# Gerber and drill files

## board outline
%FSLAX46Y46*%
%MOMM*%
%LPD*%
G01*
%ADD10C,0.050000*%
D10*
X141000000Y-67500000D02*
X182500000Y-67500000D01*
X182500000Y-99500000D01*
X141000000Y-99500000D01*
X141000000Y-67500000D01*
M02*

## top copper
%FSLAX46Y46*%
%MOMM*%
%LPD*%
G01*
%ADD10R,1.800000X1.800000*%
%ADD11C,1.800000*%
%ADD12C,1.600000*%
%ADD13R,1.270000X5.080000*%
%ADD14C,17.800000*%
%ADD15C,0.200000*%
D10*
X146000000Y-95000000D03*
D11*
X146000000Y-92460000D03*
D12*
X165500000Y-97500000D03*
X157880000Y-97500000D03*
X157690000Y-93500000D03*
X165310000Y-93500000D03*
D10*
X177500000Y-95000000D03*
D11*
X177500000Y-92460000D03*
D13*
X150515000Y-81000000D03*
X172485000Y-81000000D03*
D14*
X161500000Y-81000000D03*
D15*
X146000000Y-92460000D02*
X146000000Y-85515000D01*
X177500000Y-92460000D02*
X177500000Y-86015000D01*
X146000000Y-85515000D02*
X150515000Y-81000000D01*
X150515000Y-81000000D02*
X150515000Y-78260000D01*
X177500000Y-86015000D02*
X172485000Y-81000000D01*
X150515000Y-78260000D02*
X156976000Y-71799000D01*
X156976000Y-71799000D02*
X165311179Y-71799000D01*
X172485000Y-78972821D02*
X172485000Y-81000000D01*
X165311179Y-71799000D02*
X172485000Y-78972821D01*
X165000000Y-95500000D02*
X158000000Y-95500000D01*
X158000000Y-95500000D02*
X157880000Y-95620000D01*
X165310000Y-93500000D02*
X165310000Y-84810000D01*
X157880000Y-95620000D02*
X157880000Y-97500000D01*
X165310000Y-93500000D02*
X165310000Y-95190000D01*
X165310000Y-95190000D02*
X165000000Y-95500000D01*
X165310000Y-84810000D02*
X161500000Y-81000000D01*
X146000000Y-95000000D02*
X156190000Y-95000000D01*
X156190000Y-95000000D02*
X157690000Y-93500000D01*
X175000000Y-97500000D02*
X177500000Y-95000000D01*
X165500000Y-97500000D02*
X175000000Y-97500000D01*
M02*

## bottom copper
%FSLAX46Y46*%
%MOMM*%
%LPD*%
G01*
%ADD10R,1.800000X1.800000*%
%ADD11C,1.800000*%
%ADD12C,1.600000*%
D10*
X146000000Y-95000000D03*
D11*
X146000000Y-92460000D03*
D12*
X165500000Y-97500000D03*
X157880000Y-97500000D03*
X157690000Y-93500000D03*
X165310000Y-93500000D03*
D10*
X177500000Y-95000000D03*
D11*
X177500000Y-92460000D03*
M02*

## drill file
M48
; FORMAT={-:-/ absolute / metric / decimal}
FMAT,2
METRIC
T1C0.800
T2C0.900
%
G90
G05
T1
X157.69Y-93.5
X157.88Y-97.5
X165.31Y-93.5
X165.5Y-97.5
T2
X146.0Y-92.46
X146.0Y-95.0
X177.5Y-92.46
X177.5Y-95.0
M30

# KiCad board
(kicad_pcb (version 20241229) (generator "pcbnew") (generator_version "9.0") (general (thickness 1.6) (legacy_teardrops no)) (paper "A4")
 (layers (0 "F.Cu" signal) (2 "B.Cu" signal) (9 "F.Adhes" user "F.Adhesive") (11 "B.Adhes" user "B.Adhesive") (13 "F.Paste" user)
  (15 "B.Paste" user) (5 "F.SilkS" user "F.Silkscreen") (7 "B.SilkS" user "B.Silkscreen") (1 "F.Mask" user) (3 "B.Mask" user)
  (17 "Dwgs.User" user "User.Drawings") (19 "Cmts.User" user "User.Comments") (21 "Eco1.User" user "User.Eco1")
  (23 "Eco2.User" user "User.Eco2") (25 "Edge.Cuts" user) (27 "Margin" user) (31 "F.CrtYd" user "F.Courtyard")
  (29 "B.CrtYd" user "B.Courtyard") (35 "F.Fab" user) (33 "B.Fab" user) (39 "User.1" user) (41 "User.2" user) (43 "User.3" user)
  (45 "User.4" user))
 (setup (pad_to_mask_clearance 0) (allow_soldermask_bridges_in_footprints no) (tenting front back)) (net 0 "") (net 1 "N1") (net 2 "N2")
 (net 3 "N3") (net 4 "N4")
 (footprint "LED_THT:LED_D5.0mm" (layer "F.Cu") (at 146 95 90)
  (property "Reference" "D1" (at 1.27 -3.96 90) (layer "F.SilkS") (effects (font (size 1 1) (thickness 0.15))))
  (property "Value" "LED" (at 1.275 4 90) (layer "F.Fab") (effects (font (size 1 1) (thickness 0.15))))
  (pad "1" thru_hole rect (at 0 0 90) (size 1.8 1.8) (drill 0.9) (layers "*.Cu" "*.Mask") (remove_unused_layers no) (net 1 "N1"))
  (pad "2" thru_hole circle (at 2.54 0 90) (size 1.8 1.8) (drill 0.9) (layers "*.Cu" "*.Mask") (remove_unused_layers no) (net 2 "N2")))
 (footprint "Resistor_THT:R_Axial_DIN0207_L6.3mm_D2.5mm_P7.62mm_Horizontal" (layer "F.Cu") (at 165.5 97.5 180)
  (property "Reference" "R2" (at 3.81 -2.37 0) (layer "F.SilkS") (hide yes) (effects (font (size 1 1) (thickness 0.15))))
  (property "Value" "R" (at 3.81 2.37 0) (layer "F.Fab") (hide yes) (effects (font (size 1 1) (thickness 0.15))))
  (pad "1" thru_hole circle (at 0 0 180) (size 1.6 1.6) (drill 0.8) (layers "*.Cu" "*.Mask") (remove_unused_layers no) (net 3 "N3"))
  (pad "2" thru_hole circle (at 7.62 0 180) (size 1.6 1.6) (drill 0.8) (layers "*.Cu" "*.Mask") (remove_unused_layers no) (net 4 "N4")))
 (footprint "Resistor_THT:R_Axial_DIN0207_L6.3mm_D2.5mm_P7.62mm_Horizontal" (layer "F.Cu") (at 157.69 93.5)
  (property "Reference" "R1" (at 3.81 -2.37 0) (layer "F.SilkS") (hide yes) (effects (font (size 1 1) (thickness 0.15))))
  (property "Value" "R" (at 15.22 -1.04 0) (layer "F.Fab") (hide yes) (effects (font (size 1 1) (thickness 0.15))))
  (pad "1" thru_hole circle (at 0 0) (size 1.6 1.6) (drill 0.8) (layers "*.Cu" "*.Mask") (remove_unused_layers no) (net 1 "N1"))
  (pad "2" thru_hole circle (at 7.62 0) (size 1.6 1.6) (drill 0.8) (layers "*.Cu" "*.Mask") (remove_unused_layers no) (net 4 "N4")))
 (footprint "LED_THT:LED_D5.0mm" (layer "F.Cu") (at 177.5 95 90)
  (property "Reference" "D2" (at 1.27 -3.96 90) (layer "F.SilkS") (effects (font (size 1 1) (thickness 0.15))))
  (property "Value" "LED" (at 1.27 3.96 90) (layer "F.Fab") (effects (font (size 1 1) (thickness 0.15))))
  (pad "1" thru_hole rect (at 0 0 90) (size 1.8 1.8) (drill 0.9) (layers "*.Cu" "*.Mask") (remove_unused_layers no) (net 3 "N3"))
  (pad "2" thru_hole circle (at 2.54 0 90) (size 1.8 1.8) (drill 0.9) (layers "*.Cu" "*.Mask") (remove_unused_layers no) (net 2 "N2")))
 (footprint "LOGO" (layer "F.Cu") (at 177 72.5)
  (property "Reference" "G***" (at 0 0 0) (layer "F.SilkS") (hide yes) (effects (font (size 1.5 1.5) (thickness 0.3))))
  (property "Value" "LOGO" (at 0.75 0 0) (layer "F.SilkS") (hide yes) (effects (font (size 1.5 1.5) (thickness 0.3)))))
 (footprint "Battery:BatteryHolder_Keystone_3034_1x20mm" (layer "F.Cu") (at 161.5 81)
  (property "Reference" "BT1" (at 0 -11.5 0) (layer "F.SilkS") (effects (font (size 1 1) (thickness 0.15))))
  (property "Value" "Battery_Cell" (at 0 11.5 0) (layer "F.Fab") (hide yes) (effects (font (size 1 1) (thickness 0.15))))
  (pad "1" smd rect (at -10.985 0) (size 1.27 5.08) (layers "F.Cu" "F.Mask" "F.Paste") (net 2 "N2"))
  (pad "1" smd rect (at 10.985 0) (size 1.27 5.08) (layers "F.Cu" "F.Mask" "F.Paste") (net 2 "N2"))
  (pad "2" smd circle (at 0 0) (size 17.8 17.8) (layers "F.Cu" "F.Mask") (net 4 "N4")))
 (gr_rect (start 141 67.5) (end 182.5 99.5) (stroke (width 0.05) (type default)) (fill no) (layer "Edge.Cuts"))
 (segment (start 146 92.46) (end 146 85.515) (width 0.2) (layer "F.Cu") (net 2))
 (segment (start 177.5 92.46) (end 177.5 86.015) (width 0.2) (layer "F.Cu") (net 2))
 (segment (start 146 85.515) (end 150.515 81) (width 0.2) (layer "F.Cu") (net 2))
 (segment (start 150.515 81) (end 150.515 78.26) (width 0.2) (layer "F.Cu") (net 2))
 (segment (start 177.5 86.015) (end 172.485 81) (width 0.2) (layer "F.Cu") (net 2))
 (segment (start 150.515 78.26) (end 156.976 71.799) (width 0.2) (layer "F.Cu") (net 2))
 (segment (start 156.976 71.799) (end 165.311179 71.799) (width 0.2) (layer "F.Cu") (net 2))
 (segment (start 172.485 78.972821) (end 172.485 81) (width 0.2) (layer "F.Cu") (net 2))
 (segment (start 165.311179 71.799) (end 172.485 78.972821) (width 0.2) (layer "F.Cu") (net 2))
 (segment (start 165 95.5) (end 158 95.5) (width 0.2) (layer "F.Cu") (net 4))
 (segment (start 158 95.5) (end 157.88 95.62) (width 0.2) (layer "F.Cu") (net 4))
 (segment (start 165.31 93.5) (end 165.31 84.81) (width 0.2) (layer "F.Cu") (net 4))
 (segment (start 157.88 95.62) (end 157.88 97.5) (width 0.2) (layer "F.Cu") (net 4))
 (segment (start 165.31 93.5) (end 165.31 95.19) (width 0.2) (layer "F.Cu") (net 4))
 (segment (start 165.31 95.19) (end 165 95.5) (width 0.2) (layer "F.Cu") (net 4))
 (segment (start 165.31 84.81) (end 161.5 81) (width 0.2) (layer "F.Cu") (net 4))
 (segment (start 146 95) (end 156.19 95) (width 0.2) (layer "F.Cu") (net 1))
 (segment (start 156.19 95) (end 157.69 93.5) (width 0.2) (layer "F.Cu") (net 1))
 (segment (start 175 97.5) (end 177.5 95) (width 0.2) (layer "F.Cu") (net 3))
 (segment (start 165.5 97.5) (end 175 97.5) (width 0.2) (layer "F.Cu") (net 3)))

